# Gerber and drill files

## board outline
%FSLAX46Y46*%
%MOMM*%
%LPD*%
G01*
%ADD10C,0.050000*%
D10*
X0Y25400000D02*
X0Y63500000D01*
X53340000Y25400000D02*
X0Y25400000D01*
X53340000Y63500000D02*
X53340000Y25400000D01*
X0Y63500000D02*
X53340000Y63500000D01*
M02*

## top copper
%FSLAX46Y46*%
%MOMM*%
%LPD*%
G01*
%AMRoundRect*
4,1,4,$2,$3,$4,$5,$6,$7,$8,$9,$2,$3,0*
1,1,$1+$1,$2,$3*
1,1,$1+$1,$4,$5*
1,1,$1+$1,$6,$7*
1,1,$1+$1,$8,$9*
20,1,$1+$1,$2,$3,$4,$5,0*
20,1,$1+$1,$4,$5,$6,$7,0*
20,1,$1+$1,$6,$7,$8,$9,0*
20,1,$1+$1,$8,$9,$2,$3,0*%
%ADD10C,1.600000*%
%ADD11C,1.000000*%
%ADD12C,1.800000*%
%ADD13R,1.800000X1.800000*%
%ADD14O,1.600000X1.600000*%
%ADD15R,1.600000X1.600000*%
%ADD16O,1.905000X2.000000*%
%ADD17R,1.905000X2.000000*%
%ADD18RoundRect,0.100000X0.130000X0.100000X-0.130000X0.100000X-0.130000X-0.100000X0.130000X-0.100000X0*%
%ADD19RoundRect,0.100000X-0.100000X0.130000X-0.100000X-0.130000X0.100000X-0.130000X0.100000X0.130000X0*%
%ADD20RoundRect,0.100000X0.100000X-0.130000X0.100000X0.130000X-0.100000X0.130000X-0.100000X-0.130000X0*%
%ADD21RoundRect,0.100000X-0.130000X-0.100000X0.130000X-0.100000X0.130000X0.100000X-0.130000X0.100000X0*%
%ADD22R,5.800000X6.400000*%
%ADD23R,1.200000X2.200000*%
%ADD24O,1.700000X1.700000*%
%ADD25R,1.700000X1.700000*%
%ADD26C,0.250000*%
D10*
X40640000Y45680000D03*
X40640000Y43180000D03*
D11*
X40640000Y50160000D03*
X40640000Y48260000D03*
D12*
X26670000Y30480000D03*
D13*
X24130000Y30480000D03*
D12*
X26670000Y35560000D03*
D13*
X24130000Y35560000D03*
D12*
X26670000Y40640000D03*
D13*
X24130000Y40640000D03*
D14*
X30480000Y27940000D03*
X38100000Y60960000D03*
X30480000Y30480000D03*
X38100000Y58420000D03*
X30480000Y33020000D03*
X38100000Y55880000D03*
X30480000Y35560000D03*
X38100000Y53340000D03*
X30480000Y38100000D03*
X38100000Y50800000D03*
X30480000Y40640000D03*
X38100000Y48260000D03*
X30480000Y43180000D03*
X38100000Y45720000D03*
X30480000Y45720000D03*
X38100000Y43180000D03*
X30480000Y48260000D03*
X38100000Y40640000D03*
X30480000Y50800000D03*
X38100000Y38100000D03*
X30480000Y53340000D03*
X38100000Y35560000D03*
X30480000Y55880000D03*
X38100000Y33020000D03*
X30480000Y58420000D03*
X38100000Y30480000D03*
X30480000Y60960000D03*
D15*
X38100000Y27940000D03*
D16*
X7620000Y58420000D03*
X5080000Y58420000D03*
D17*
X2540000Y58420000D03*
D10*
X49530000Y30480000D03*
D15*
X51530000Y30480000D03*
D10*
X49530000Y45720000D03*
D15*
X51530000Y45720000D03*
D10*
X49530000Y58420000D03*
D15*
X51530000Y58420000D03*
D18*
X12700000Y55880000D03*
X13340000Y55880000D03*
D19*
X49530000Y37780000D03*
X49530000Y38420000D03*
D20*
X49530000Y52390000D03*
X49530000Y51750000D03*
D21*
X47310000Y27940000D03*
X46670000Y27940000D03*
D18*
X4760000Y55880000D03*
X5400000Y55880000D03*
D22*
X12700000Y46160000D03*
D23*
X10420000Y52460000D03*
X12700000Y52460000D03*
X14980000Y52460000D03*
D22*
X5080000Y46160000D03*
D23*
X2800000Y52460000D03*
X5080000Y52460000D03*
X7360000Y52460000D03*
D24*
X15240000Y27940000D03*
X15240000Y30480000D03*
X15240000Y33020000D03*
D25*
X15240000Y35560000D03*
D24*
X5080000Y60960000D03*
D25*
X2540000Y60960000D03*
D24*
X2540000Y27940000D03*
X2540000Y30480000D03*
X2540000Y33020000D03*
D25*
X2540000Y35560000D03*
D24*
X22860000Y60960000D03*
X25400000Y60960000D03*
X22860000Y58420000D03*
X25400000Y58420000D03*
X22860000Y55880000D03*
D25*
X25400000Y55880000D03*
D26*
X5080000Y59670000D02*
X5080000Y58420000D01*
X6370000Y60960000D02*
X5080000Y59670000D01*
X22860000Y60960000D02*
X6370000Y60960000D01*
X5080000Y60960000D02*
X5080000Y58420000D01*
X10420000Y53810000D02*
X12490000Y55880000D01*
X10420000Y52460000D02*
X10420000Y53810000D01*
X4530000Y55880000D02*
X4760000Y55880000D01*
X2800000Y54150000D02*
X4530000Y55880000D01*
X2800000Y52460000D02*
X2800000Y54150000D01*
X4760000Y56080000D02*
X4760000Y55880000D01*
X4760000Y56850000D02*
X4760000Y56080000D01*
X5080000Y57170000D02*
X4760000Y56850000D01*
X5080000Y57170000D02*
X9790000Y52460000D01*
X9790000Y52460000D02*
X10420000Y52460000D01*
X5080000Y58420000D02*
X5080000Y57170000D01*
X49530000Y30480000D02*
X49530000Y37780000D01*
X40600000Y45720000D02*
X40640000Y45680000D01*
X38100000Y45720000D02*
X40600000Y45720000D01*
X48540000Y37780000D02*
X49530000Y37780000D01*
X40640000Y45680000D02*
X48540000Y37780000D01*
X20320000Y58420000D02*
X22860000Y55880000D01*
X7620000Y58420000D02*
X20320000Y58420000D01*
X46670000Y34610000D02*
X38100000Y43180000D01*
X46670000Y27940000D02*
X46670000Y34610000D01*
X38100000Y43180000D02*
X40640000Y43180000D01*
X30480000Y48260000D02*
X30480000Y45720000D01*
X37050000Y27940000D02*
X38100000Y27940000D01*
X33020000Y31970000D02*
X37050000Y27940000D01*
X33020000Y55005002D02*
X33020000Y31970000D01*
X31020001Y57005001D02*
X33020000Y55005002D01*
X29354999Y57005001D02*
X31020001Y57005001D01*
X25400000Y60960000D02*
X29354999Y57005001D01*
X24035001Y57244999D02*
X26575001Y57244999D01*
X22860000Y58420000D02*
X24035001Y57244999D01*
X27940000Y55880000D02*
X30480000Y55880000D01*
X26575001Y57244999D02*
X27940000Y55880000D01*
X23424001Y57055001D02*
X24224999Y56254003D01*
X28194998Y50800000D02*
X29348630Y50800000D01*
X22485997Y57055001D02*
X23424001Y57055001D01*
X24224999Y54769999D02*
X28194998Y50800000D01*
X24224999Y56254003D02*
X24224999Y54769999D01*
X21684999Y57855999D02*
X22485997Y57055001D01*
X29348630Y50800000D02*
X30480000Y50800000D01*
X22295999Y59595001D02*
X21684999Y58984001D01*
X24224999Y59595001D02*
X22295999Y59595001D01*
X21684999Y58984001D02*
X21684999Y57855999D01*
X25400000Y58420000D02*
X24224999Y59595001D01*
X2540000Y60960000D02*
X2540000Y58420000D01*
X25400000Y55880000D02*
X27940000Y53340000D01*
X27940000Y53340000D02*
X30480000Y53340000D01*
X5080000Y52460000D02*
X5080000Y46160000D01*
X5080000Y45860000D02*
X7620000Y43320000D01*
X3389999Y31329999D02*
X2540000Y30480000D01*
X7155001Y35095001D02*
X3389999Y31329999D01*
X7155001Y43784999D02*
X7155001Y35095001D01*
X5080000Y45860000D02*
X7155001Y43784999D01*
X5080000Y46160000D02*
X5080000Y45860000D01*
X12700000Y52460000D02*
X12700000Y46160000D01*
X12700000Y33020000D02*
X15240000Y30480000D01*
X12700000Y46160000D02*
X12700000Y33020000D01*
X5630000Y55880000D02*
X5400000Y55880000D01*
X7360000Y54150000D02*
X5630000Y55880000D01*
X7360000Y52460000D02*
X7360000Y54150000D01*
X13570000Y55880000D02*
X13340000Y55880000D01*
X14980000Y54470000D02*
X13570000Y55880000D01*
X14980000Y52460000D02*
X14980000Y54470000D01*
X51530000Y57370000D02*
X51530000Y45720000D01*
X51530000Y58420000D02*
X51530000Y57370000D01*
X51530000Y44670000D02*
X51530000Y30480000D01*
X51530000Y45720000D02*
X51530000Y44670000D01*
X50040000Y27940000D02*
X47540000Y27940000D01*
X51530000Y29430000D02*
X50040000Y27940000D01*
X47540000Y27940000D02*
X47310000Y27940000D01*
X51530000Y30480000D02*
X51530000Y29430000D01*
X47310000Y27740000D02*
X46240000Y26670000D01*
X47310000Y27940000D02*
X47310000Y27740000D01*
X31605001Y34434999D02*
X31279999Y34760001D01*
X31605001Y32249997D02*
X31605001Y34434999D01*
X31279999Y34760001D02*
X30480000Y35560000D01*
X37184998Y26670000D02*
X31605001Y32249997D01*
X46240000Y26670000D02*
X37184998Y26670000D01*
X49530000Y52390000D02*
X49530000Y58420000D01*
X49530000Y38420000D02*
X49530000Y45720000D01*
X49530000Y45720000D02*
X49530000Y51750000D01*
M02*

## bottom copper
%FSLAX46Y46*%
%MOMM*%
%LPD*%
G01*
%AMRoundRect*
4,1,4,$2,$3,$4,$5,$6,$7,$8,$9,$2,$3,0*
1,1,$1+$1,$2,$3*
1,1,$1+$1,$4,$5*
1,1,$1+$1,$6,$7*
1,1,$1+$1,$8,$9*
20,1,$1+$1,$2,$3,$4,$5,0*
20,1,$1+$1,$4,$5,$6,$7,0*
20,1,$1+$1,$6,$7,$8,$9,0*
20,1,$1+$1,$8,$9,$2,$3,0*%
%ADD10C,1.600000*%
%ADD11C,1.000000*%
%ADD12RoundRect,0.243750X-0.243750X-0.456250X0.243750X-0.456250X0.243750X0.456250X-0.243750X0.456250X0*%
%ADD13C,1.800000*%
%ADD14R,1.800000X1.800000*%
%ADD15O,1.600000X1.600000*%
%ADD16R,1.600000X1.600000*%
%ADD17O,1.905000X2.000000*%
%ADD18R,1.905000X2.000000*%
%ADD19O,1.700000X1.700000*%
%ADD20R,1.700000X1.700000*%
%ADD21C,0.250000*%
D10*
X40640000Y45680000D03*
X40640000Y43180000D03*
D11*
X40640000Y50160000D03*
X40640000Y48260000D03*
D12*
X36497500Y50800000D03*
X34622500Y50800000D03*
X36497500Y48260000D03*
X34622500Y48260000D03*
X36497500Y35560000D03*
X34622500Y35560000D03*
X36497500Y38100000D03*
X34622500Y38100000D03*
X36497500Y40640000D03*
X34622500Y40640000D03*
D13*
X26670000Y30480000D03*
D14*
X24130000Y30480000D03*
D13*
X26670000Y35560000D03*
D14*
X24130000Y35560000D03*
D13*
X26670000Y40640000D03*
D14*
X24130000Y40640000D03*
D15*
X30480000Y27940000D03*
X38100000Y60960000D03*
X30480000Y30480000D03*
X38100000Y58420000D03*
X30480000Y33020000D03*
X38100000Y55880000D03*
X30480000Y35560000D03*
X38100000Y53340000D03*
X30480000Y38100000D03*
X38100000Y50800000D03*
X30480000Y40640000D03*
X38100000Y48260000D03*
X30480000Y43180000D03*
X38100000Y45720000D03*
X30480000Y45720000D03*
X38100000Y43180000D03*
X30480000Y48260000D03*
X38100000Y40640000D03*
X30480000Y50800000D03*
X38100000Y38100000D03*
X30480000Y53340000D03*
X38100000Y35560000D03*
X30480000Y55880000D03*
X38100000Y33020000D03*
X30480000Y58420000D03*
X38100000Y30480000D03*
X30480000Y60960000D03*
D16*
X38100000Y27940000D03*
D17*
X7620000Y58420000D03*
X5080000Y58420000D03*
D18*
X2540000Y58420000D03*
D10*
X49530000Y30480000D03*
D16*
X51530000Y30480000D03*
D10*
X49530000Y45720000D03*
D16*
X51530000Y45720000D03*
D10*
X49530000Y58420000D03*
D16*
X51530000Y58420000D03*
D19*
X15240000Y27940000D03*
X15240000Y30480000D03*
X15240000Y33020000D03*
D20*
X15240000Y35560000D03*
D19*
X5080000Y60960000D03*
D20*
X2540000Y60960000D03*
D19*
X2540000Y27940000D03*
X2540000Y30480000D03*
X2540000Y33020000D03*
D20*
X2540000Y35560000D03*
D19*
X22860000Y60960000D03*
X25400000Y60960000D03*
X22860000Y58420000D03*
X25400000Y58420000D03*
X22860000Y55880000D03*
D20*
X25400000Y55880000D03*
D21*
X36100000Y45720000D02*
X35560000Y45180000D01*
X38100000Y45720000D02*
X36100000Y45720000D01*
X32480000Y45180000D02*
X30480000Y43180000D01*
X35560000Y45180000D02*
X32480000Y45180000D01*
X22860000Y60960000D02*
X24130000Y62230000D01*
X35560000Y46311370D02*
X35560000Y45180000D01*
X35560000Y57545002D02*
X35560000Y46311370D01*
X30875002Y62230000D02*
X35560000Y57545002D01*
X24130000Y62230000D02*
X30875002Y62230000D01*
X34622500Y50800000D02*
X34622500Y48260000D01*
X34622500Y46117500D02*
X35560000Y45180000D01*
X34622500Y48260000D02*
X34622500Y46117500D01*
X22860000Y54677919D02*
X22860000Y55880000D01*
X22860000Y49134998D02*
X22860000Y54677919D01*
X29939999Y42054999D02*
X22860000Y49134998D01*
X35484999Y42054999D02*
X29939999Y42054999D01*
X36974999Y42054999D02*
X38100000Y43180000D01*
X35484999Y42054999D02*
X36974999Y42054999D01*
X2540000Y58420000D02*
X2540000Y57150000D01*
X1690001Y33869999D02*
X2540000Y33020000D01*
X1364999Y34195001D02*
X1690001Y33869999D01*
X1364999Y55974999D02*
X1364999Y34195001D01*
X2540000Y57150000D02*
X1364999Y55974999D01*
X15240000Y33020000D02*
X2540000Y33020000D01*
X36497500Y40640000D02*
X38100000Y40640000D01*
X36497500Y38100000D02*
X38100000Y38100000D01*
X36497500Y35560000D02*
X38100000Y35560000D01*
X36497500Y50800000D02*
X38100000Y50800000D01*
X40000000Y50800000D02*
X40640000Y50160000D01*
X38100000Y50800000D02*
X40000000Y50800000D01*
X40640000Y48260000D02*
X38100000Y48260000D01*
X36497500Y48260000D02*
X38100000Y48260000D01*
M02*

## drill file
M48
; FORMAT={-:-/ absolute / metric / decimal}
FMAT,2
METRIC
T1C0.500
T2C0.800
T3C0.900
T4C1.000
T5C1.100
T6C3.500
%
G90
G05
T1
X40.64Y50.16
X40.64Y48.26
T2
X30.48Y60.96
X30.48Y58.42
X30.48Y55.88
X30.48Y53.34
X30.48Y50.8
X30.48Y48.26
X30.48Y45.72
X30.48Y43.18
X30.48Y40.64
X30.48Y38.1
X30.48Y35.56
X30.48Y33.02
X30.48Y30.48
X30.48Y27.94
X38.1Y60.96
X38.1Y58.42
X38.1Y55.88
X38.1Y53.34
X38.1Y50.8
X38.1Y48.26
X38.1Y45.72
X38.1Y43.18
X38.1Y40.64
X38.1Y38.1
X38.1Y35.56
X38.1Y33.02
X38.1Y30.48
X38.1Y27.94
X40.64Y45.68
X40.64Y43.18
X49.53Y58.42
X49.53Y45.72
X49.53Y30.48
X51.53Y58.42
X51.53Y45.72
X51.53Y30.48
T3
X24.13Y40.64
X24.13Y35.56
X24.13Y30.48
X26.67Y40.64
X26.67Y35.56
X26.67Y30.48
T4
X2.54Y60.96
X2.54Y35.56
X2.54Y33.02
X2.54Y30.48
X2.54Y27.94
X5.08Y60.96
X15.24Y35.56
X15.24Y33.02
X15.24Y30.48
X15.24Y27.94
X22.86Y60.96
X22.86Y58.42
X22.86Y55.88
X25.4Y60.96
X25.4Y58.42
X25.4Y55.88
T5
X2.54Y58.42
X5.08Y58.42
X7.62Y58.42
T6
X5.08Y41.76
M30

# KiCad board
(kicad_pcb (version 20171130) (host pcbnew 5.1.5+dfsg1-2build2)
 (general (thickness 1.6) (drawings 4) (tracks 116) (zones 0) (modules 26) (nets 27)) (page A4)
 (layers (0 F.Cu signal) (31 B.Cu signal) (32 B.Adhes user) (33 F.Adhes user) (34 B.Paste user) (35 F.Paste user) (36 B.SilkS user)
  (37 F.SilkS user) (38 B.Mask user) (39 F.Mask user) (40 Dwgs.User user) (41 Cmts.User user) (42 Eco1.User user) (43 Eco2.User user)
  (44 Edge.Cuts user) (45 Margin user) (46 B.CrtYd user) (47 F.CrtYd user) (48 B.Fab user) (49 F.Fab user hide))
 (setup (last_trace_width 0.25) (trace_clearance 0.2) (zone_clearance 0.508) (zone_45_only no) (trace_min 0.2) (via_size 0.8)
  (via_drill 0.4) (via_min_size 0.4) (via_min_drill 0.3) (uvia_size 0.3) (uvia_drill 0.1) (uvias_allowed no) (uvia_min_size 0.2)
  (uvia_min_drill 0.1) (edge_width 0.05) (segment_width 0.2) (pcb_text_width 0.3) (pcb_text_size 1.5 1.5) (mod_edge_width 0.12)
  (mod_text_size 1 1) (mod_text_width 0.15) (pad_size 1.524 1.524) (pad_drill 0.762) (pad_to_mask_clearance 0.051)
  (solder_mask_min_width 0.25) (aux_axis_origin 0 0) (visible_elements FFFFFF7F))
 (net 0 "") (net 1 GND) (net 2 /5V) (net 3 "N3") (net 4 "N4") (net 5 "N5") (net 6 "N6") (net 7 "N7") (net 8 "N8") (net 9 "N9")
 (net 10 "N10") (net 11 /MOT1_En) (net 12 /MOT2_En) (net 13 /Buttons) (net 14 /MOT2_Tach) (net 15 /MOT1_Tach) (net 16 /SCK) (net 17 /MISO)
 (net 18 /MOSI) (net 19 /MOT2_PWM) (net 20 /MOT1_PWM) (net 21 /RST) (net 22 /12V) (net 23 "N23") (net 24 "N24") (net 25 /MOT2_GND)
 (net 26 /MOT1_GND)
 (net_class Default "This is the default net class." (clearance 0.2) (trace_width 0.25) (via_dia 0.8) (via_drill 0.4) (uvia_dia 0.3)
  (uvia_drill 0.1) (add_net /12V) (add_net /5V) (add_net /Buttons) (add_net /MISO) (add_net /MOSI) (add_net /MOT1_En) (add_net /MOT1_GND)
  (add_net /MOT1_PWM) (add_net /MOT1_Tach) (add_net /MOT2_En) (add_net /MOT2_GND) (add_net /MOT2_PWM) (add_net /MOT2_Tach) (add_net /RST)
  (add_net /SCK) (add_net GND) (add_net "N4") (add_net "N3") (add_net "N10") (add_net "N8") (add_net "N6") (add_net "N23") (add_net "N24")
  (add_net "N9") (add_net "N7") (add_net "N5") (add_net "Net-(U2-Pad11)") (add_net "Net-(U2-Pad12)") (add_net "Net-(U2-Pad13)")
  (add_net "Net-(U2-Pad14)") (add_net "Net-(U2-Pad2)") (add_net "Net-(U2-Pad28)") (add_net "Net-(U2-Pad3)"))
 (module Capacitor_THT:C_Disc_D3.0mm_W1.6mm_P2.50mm (layer F.Cu) (at 40.64 -43.18 90)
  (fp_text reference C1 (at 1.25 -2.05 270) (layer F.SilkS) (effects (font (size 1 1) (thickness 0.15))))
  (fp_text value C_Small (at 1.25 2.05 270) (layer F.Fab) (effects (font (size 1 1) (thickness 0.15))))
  (pad 2 thru_hole circle (at 2.5 0 90) (size 1.6 1.6) (drill 0.8) (layers *.Cu *.Mask) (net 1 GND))
  (pad 1 thru_hole circle (at 0 0 90) (size 1.6 1.6) (drill 0.8) (layers *.Cu *.Mask) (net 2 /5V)))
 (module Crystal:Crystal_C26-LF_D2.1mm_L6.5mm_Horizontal (layer F.Cu) (at 40.64 -48.26 90)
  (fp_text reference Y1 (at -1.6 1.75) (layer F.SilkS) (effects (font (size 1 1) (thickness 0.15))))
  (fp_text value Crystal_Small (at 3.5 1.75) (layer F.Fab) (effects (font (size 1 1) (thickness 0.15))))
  (pad 2 thru_hole circle (at 1.9 0 90) (size 1 1) (drill 0.5) (layers *.Cu *.Mask) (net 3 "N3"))
  (pad 1 thru_hole circle (at 0 0 90) (size 1 1) (drill 0.5) (layers *.Cu *.Mask) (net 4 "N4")))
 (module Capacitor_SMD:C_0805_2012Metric (layer B.Cu) (at 35.56 -50.8)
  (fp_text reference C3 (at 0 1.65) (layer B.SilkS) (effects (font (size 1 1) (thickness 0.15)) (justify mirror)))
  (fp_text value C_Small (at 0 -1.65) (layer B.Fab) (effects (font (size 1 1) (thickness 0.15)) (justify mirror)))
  (pad 2 smd roundrect (at 0.9375 0) (size 0.975 1.4) (layers B.Cu B.Paste B.Mask) (roundrect_rratio 0.25) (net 3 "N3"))
  (pad 1 smd roundrect (at -0.9375 0) (size 0.975 1.4) (layers B.Cu B.Paste B.Mask) (roundrect_rratio 0.25) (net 1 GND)))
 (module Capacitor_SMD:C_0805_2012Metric (layer B.Cu) (at 35.56 -48.26)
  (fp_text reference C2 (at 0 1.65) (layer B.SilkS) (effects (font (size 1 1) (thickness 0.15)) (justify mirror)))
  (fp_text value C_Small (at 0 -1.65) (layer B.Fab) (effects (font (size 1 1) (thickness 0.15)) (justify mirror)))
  (pad 2 smd roundrect (at 0.9375 0) (size 0.975 1.4) (layers B.Cu B.Paste B.Mask) (roundrect_rratio 0.25) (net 4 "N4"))
  (pad 1 smd roundrect (at -0.9375 0) (size 0.975 1.4) (layers B.Cu B.Paste B.Mask) (roundrect_rratio 0.25) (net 1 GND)))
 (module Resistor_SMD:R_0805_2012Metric (layer B.Cu) (at 35.56 -35.56)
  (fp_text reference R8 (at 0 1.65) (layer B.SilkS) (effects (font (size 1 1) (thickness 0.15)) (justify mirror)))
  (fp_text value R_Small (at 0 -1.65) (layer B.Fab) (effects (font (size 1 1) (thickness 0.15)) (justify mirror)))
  (pad 2 smd roundrect (at 0.9375 0) (size 0.975 1.4) (layers B.Cu B.Paste B.Mask) (roundrect_rratio 0.25) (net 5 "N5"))
  (pad 1 smd roundrect (at -0.9375 0) (size 0.975 1.4) (layers B.Cu B.Paste B.Mask) (roundrect_rratio 0.25) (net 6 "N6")))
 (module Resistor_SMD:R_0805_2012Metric (layer B.Cu) (at 35.56 -38.1)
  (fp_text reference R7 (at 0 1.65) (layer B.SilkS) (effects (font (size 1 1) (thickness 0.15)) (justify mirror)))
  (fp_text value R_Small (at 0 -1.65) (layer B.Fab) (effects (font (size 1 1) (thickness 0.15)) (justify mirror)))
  (pad 2 smd roundrect (at 0.9375 0) (size 0.975 1.4) (layers B.Cu B.Paste B.Mask) (roundrect_rratio 0.25) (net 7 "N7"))
  (pad 1 smd roundrect (at -0.9375 0) (size 0.975 1.4) (layers B.Cu B.Paste B.Mask) (roundrect_rratio 0.25) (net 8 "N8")))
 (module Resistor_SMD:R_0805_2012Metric (layer B.Cu) (at 35.56 -40.64)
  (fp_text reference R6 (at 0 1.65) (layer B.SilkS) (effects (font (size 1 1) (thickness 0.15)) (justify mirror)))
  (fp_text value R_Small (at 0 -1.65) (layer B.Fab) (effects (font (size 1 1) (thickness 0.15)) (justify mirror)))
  (pad 2 smd roundrect (at 0.9375 0) (size 0.975 1.4) (layers B.Cu B.Paste B.Mask) (roundrect_rratio 0.25) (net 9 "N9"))
  (pad 1 smd roundrect (at -0.9375 0) (size 0.975 1.4) (layers B.Cu B.Paste B.Mask) (roundrect_rratio 0.25) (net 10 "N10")))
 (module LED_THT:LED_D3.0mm (layer B.Cu) (at 24.13 -30.48)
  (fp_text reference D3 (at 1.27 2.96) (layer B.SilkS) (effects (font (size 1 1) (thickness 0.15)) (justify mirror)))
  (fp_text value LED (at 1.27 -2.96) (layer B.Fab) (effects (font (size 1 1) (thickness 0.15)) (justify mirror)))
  (pad 2 thru_hole circle (at 2.54 0) (size 1.8 1.8) (drill 0.9) (layers *.Cu *.Mask) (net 6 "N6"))
  (pad 1 thru_hole rect (at 0 0) (size 1.8 1.8) (drill 0.9) (layers *.Cu *.Mask) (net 1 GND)))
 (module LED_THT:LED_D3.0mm (layer B.Cu) (at 24.13 -35.56)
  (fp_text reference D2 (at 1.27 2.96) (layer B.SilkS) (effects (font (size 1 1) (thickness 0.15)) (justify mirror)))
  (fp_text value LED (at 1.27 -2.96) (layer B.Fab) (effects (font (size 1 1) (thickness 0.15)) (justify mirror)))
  (pad 2 thru_hole circle (at 2.54 0) (size 1.8 1.8) (drill 0.9) (layers *.Cu *.Mask) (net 8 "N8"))
  (pad 1 thru_hole rect (at 0 0) (size 1.8 1.8) (drill 0.9) (layers *.Cu *.Mask) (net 1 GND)))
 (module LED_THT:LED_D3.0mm (layer B.Cu) (at 24.13 -40.64)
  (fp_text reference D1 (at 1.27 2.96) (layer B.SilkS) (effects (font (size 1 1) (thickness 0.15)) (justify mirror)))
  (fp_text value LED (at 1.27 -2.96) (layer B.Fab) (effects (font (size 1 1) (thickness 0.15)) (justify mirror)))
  (pad 2 thru_hole circle (at 2.54 0) (size 1.8 1.8) (drill 0.9) (layers *.Cu *.Mask) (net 10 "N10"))
  (pad 1 thru_hole rect (at 0 0) (size 1.8 1.8) (drill 0.9) (layers *.Cu *.Mask) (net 1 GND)))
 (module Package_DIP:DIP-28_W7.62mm (layer F.Cu) (at 38.1 -27.94 180)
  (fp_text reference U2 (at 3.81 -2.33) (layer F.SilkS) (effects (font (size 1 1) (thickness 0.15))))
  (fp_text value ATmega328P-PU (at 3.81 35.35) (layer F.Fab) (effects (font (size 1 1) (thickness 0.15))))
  (pad 28 thru_hole oval (at 7.62 0 180) (size 1.6 1.6) (drill 0.8) (layers *.Cu *.Mask))
  (pad 14 thru_hole oval (at 0 33.02 180) (size 1.6 1.6) (drill 0.8) (layers *.Cu *.Mask))
  (pad 27 thru_hole oval (at 7.62 2.54 180) (size 1.6 1.6) (drill 0.8) (layers *.Cu *.Mask) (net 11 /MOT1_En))
  (pad 13 thru_hole oval (at 0 30.48 180) (size 1.6 1.6) (drill 0.8) (layers *.Cu *.Mask))
  (pad 26 thru_hole oval (at 7.62 5.08 180) (size 1.6 1.6) (drill 0.8) (layers *.Cu *.Mask) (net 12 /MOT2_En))
  (pad 12 thru_hole oval (at 0 27.94 180) (size 1.6 1.6) (drill 0.8) (layers *.Cu *.Mask))
  (pad 25 thru_hole oval (at 7.62 7.62 180) (size 1.6 1.6) (drill 0.8) (layers *.Cu *.Mask) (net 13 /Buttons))
  (pad 11 thru_hole oval (at 0 25.4 180) (size 1.6 1.6) (drill 0.8) (layers *.Cu *.Mask))
  (pad 24 thru_hole oval (at 7.62 10.16 180) (size 1.6 1.6) (drill 0.8) (layers *.Cu *.Mask) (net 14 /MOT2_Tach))
  (pad 10 thru_hole oval (at 0 22.86 180) (size 1.6 1.6) (drill 0.8) (layers *.Cu *.Mask) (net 3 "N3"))
  (pad 23 thru_hole oval (at 7.62 12.7 180) (size 1.6 1.6) (drill 0.8) (layers *.Cu *.Mask) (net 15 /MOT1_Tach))
  (pad 9 thru_hole oval (at 0 20.32 180) (size 1.6 1.6) (drill 0.8) (layers *.Cu *.Mask) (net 4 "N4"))
  (pad 22 thru_hole oval (at 7.62 15.24 180) (size 1.6 1.6) (drill 0.8) (layers *.Cu *.Mask) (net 1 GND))
  (pad 8 thru_hole oval (at 0 17.78 180) (size 1.6 1.6) (drill 0.8) (layers *.Cu *.Mask) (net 1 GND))
  (pad 21 thru_hole oval (at 7.62 17.78 180) (size 1.6 1.6) (drill 0.8) (layers *.Cu *.Mask) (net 2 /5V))
  (pad 7 thru_hole oval (at 0 15.24 180) (size 1.6 1.6) (drill 0.8) (layers *.Cu *.Mask) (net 2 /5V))
  (pad 20 thru_hole oval (at 7.62 20.32 180) (size 1.6 1.6) (drill 0.8) (layers *.Cu *.Mask) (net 2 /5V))
  (pad 6 thru_hole oval (at 0 12.7 180) (size 1.6 1.6) (drill 0.8) (layers *.Cu *.Mask) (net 9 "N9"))
  (pad 19 thru_hole oval (at 7.62 22.86 180) (size 1.6 1.6) (drill 0.8) (layers *.Cu *.Mask) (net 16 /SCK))
  (pad 5 thru_hole oval (at 0 10.16 180) (size 1.6 1.6) (drill 0.8) (layers *.Cu *.Mask) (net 7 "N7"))
  (pad 18 thru_hole oval (at 7.62 25.4 180) (size 1.6 1.6) (drill 0.8) (layers *.Cu *.Mask) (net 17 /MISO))
  (pad 4 thru_hole oval (at 0 7.62 180) (size 1.6 1.6) (drill 0.8) (layers *.Cu *.Mask) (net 5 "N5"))
  (pad 17 thru_hole oval (at 7.62 27.94 180) (size 1.6 1.6) (drill 0.8) (layers *.Cu *.Mask) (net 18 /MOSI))
  (pad 3 thru_hole oval (at 0 5.08 180) (size 1.6 1.6) (drill 0.8) (layers *.Cu *.Mask))
  (pad 16 thru_hole oval (at 7.62 30.48 180) (size 1.6 1.6) (drill 0.8) (layers *.Cu *.Mask) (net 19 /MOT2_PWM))
  (pad 2 thru_hole oval (at 0 2.54 180) (size 1.6 1.6) (drill 0.8) (layers *.Cu *.Mask))
  (pad 15 thru_hole oval (at 7.62 33.02 180) (size 1.6 1.6) (drill 0.8) (layers *.Cu *.Mask) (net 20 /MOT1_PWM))
  (pad 1 thru_hole rect (at 0 0 180) (size 1.6 1.6) (drill 0.8) (layers *.Cu *.Mask) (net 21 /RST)))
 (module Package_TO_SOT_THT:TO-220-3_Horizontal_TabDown (layer B.Cu) (at 2.54 -58.42)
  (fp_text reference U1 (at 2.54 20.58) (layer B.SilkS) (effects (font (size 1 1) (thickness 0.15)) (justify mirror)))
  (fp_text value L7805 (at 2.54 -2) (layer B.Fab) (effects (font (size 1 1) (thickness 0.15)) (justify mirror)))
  (pad 3 thru_hole oval (at 5.08 0) (size 1.905 2) (drill 1.1) (layers *.Cu *.Mask) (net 2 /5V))
  (pad 2 thru_hole oval (at 2.54 0) (size 1.905 2) (drill 1.1) (layers *.Cu *.Mask) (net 1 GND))
  (pad 1 thru_hole rect (at 0 0) (size 1.905 2) (drill 1.1) (layers *.Cu *.Mask) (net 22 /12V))
  (pad "" np_thru_hole oval (at 2.54 16.66) (size 3.5 3.5) (drill 3.5) (layers *.Cu *.Mask)))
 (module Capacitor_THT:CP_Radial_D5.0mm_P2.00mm (layer B.Cu) (at 51.53 -30.48 180)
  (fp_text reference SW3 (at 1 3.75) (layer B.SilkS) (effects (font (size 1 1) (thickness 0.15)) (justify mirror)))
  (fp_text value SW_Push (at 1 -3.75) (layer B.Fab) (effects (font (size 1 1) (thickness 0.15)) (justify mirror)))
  (pad 2 thru_hole circle (at 2 0 180) (size 1.6 1.6) (drill 0.8) (layers *.Cu *.Mask) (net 1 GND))
  (pad 1 thru_hole rect (at 0 0 180) (size 1.6 1.6) (drill 0.8) (layers *.Cu *.Mask) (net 13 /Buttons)))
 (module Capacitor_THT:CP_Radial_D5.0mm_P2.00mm (layer B.Cu) (at 51.53 -45.72 180)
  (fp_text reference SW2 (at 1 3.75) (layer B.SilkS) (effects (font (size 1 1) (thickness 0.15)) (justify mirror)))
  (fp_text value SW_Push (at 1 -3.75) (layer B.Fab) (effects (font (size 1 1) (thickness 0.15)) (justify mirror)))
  (pad 2 thru_hole circle (at 2 0 180) (size 1.6 1.6) (drill 0.8) (layers *.Cu *.Mask) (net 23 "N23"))
  (pad 1 thru_hole rect (at 0 0 180) (size 1.6 1.6) (drill 0.8) (layers *.Cu *.Mask) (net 13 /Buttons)))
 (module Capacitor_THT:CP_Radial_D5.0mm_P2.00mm (layer B.Cu) (at 51.53 -58.42 180)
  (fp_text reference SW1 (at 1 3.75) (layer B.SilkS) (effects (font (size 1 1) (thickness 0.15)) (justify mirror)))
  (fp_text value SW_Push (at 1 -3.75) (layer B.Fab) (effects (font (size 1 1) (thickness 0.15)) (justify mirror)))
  (pad 2 thru_hole circle (at 2 0 180) (size 1.6 1.6) (drill 0.8) (layers *.Cu *.Mask) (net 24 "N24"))
  (pad 1 thru_hole rect (at 0 0 180) (size 1.6 1.6) (drill 0.8) (layers *.Cu *.Mask) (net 13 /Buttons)))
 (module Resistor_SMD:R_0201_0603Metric (layer F.Cu) (at 13.02 -55.88 180)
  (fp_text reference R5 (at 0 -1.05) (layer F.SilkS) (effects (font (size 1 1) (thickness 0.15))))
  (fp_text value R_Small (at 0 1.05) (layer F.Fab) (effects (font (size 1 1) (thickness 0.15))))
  (pad 2 smd roundrect (at 0.32 0 180) (size 0.46 0.4) (layers F.Cu F.Mask) (roundrect_rratio 0.25) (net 1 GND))
  (pad 1 smd roundrect (at -0.32 0 180) (size 0.46 0.4) (layers F.Cu F.Mask) (roundrect_rratio 0.25) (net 12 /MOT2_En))
  (pad "" smd roundrect (at 0.345 0 180) (size 0.318 0.36) (layers F.Paste) (roundrect_rratio 0.25))
  (pad "" smd roundrect (at -0.345 0 180) (size 0.318 0.36) (layers F.Paste) (roundrect_rratio 0.25)))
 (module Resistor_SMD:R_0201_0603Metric (layer F.Cu) (at 49.53 -38.1 270)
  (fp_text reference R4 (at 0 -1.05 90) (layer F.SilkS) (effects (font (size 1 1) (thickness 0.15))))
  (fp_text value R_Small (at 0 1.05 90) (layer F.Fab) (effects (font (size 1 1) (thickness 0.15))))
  (pad 2 smd roundrect (at 0.32 0 270) (size 0.46 0.4) (layers F.Cu F.Mask) (roundrect_rratio 0.25) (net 1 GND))
  (pad 1 smd roundrect (at -0.32 0 270) (size 0.46 0.4) (layers F.Cu F.Mask) (roundrect_rratio 0.25) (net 23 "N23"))
  (pad "" smd roundrect (at 0.345 0 270) (size 0.318 0.36) (layers F.Paste) (roundrect_rratio 0.25))
  (pad "" smd roundrect (at -0.345 0 270) (size 0.318 0.36) (layers F.Paste) (roundrect_rratio 0.25)))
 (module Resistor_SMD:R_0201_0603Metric (layer F.Cu) (at 49.53 -52.07 90)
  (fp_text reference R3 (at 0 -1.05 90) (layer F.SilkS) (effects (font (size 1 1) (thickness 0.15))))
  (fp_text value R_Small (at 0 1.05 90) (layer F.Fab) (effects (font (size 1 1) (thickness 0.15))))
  (pad 2 smd roundrect (at 0.32 0 90) (size 0.46 0.4) (layers F.Cu F.Mask) (roundrect_rratio 0.25) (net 24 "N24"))
  (pad 1 smd roundrect (at -0.32 0 90) (size 0.46 0.4) (layers F.Cu F.Mask) (roundrect_rratio 0.25) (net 23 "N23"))
  (pad "" smd roundrect (at 0.345 0 90) (size 0.318 0.36) (layers F.Paste) (roundrect_rratio 0.25))
  (pad "" smd roundrect (at -0.345 0 90) (size 0.318 0.36) (layers F.Paste) (roundrect_rratio 0.25)))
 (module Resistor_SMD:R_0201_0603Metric (layer F.Cu) (at 46.99 -27.94)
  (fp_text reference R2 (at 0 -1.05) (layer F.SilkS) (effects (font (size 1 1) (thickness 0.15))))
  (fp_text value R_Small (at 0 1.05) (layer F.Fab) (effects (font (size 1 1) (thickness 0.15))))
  (pad 2 smd roundrect (at 0.32 0) (size 0.46 0.4) (layers F.Cu F.Mask) (roundrect_rratio 0.25) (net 13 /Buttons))
  (pad 1 smd roundrect (at -0.32 0) (size 0.46 0.4) (layers F.Cu F.Mask) (roundrect_rratio 0.25) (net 2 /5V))
  (pad "" smd roundrect (at 0.345 0) (size 0.318 0.36) (layers F.Paste) (roundrect_rratio 0.25))
  (pad "" smd roundrect (at -0.345 0) (size 0.318 0.36) (layers F.Paste) (roundrect_rratio 0.25)))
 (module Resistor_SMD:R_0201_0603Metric (layer F.Cu) (at 5.08 -55.88 180)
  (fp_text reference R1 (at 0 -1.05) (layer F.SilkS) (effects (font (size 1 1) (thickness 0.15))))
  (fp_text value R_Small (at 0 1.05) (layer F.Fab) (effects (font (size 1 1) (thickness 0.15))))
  (pad 2 smd roundrect (at 0.32 0 180) (size 0.46 0.4) (layers F.Cu F.Mask) (roundrect_rratio 0.25) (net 1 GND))
  (pad 1 smd roundrect (at -0.32 0 180) (size 0.46 0.4) (layers F.Cu F.Mask) (roundrect_rratio 0.25) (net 11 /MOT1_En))
  (pad "" smd roundrect (at 0.345 0 180) (size 0.318 0.36) (layers F.Paste) (roundrect_rratio 0.25))
  (pad "" smd roundrect (at -0.345 0 180) (size 0.318 0.36) (layers F.Paste) (roundrect_rratio 0.25)))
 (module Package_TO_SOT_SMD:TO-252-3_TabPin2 (layer F.Cu) (at 12.7 -48.26 270)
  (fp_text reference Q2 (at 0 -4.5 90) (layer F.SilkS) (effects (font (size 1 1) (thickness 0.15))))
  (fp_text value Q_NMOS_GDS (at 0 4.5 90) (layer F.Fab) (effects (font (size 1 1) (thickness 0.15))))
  (pad "" smd rect (at 0.425 1.525 270) (size 3.05 2.75) (layers F.Paste))
  (pad "" smd rect (at 3.775 -1.525 270) (size 3.05 2.75) (layers F.Paste))
  (pad "" smd rect (at 0.425 -1.525 270) (size 3.05 2.75) (layers F.Paste))
  (pad "" smd rect (at 3.775 1.525 270) (size 3.05 2.75) (layers F.Paste))
  (pad 2 smd rect (at 2.1 0 270) (size 6.4 5.8) (layers F.Cu F.Mask) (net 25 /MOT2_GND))
  (pad 3 smd rect (at -4.2 2.28 270) (size 2.2 1.2) (layers F.Cu F.Paste F.Mask) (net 1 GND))
  (pad 2 smd rect (at -4.2 0 270) (size 2.2 1.2) (layers F.Cu F.Paste F.Mask) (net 25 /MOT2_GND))
  (pad 1 smd rect (at -4.2 -2.28 270) (size 2.2 1.2) (layers F.Cu F.Paste F.Mask) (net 12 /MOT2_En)))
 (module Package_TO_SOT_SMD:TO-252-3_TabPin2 (layer F.Cu) (at 5.08 -48.26 270)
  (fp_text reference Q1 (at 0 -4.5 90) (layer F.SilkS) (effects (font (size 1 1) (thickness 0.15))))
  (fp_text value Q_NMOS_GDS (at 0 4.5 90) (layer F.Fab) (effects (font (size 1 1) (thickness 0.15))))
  (pad "" smd rect (at 0.425 1.525 270) (size 3.05 2.75) (layers F.Paste))
  (pad "" smd rect (at 3.775 -1.525 270) (size 3.05 2.75) (layers F.Paste))
  (pad "" smd rect (at 0.425 -1.525 270) (size 3.05 2.75) (layers F.Paste))
  (pad "" smd rect (at 3.775 1.525 270) (size 3.05 2.75) (layers F.Paste))
  (pad 2 smd rect (at 2.1 0 270) (size 6.4 5.8) (layers F.Cu F.Mask) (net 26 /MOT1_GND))
  (pad 3 smd rect (at -4.2 2.28 270) (size 2.2 1.2) (layers F.Cu F.Paste F.Mask) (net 1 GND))
  (pad 2 smd rect (at -4.2 0 270) (size 2.2 1.2) (layers F.Cu F.Paste F.Mask) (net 26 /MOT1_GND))
  (pad 1 smd rect (at -4.2 -2.28 270) (size 2.2 1.2) (layers F.Cu F.Paste F.Mask) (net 11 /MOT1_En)))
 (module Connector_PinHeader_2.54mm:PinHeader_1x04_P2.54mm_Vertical (layer F.Cu) (at 15.24 -35.56)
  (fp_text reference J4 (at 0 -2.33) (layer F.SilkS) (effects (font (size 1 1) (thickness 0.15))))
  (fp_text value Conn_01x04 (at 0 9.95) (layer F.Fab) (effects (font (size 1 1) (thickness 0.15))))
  (pad 4 thru_hole oval (at 0 7.62) (size 1.7 1.7) (drill 1) (layers *.Cu *.Mask) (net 19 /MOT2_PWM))
  (pad 3 thru_hole oval (at 0 5.08) (size 1.7 1.7) (drill 1) (layers *.Cu *.Mask) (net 25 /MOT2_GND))
  (pad 2 thru_hole oval (at 0 2.54) (size 1.7 1.7) (drill 1) (layers *.Cu *.Mask) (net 22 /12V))
  (pad 1 thru_hole rect (at 0 0) (size 1.7 1.7) (drill 1) (layers *.Cu *.Mask) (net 14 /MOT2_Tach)))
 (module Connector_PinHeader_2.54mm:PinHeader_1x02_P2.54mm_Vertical (layer F.Cu) (at 2.54 -60.96 90)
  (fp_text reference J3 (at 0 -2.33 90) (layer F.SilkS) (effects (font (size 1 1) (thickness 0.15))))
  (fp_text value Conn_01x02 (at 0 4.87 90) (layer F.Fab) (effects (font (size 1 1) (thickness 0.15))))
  (pad 2 thru_hole oval (at 0 2.54 90) (size 1.7 1.7) (drill 1) (layers *.Cu *.Mask) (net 1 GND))
  (pad 1 thru_hole rect (at 0 0 90) (size 1.7 1.7) (drill 1) (layers *.Cu *.Mask) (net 22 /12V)))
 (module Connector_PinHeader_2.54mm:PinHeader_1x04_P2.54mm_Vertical (layer F.Cu) (at 2.54 -35.56)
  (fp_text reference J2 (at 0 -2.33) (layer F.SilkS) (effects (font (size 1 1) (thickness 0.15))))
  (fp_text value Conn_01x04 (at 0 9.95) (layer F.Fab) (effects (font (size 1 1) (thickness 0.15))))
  (pad 4 thru_hole oval (at 0 7.62) (size 1.7 1.7) (drill 1) (layers *.Cu *.Mask) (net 20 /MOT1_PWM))
  (pad 3 thru_hole oval (at 0 5.08) (size 1.7 1.7) (drill 1) (layers *.Cu *.Mask) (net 26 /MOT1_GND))
  (pad 2 thru_hole oval (at 0 2.54) (size 1.7 1.7) (drill 1) (layers *.Cu *.Mask) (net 22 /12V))
  (pad 1 thru_hole rect (at 0 0) (size 1.7 1.7) (drill 1) (layers *.Cu *.Mask) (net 15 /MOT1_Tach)))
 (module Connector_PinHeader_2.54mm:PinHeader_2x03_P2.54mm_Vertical (layer F.Cu) (at 25.4 -55.88 180)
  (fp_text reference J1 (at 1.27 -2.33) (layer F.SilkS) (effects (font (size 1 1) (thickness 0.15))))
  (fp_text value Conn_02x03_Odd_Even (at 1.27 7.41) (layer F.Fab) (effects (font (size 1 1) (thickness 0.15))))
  (pad 6 thru_hole oval (at 2.54 5.08 180) (size 1.7 1.7) (drill 1) (layers *.Cu *.Mask) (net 1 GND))
  (pad 5 thru_hole oval (at 0 5.08 180) (size 1.7 1.7) (drill 1) (layers *.Cu *.Mask) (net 21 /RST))
  (pad 4 thru_hole oval (at 2.54 2.54 180) (size 1.7 1.7) (drill 1) (layers *.Cu *.Mask) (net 18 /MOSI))
  (pad 3 thru_hole oval (at 0 2.54 180) (size 1.7 1.7) (drill 1) (layers *.Cu *.Mask) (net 16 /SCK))
  (pad 2 thru_hole oval (at 2.54 0 180) (size 1.7 1.7) (drill 1) (layers *.Cu *.Mask) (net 2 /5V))
  (pad 1 thru_hole rect (at 0 0 180) (size 1.7 1.7) (drill 1) (layers *.Cu *.Mask) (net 17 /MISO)))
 (gr_line (start 0 -25.4) (end 0 -63.5) (layer Edge.Cuts) (width 0.05))
 (gr_line (start 53.34 -25.4) (end 0 -25.4) (layer Edge.Cuts) (width 0.05))
 (gr_line (start 53.34 -63.5) (end 53.34 -25.4) (layer Edge.Cuts) (width 0.05))
 (gr_line (start 0 -63.5) (end 53.34 -63.5) (layer Edge.Cuts) (width 0.05))
 (segment (start 5.08 -59.67) (end 5.08 -58.42) (width 0.25) (layer F.Cu) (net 1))
 (segment (start 6.37 -60.96) (end 5.08 -59.67) (width 0.25) (layer F.Cu) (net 1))
 (segment (start 22.86 -60.96) (end 6.37 -60.96) (width 0.25) (layer F.Cu) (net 1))
 (segment (start 5.08 -60.96) (end 5.08 -58.42) (width 0.25) (layer F.Cu) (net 1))
 (segment (start 10.42 -53.81) (end 12.49 -55.88) (width 0.25) (layer F.Cu) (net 1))
 (segment (start 10.42 -52.46) (end 10.42 -53.81) (width 0.25) (layer F.Cu) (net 1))
 (segment (start 4.53 -55.88) (end 4.76 -55.88) (width 0.25) (layer F.Cu) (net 1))
 (segment (start 2.8 -54.15) (end 4.53 -55.88) (width 0.25) (layer F.Cu) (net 1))
 (segment (start 2.8 -52.46) (end 2.8 -54.15) (width 0.25) (layer F.Cu) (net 1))
 (segment (start 4.76 -56.08) (end 4.76 -55.88) (width 0.25) (layer F.Cu) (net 1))
 (segment (start 4.76 -56.85) (end 4.76 -56.08) (width 0.25) (layer F.Cu) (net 1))
 (segment (start 5.08 -57.17) (end 4.76 -56.85) (width 0.25) (layer F.Cu) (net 1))
 (segment (start 5.08 -57.17) (end 9.79 -52.46) (width 0.25) (layer F.Cu) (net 1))
 (segment (start 9.79 -52.46) (end 10.42 -52.46) (width 0.25) (layer F.Cu) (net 1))
 (segment (start 5.08 -58.42) (end 5.08 -57.17) (width 0.25) (layer F.Cu) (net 1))
 (segment (start 36.1 -45.72) (end 35.56 -45.18) (width 0.25) (layer B.Cu) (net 1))
 (segment (start 38.1 -45.72) (end 36.1 -45.72) (width 0.25) (layer B.Cu) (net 1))
 (segment (start 32.48 -45.18) (end 30.48 -43.18) (width 0.25) (layer B.Cu) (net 1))
 (segment (start 35.56 -45.18) (end 32.48 -45.18) (width 0.25) (layer B.Cu) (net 1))
 (segment (start 22.86 -60.96) (end 24.13 -62.23) (width 0.25) (layer B.Cu) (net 1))
 (segment (start 35.56 -46.31137) (end 35.56 -45.18) (width 0.25) (layer B.Cu) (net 1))
 (segment (start 35.56 -57.545002) (end 35.56 -46.31137) (width 0.25) (layer B.Cu) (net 1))
 (segment (start 30.875002 -62.23) (end 35.56 -57.545002) (width 0.25) (layer B.Cu) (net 1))
 (segment (start 24.13 -62.23) (end 30.875002 -62.23) (width 0.25) (layer B.Cu) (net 1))
 (segment (start 49.53 -30.48) (end 49.53 -37.78) (width 0.25) (layer F.Cu) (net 1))
 (segment (start 40.6 -45.72) (end 40.64 -45.68) (width 0.25) (layer F.Cu) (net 1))
 (segment (start 38.1 -45.72) (end 40.6 -45.72) (width 0.25) (layer F.Cu) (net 1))
 (segment (start 48.54 -37.78) (end 49.53 -37.78) (width 0.25) (layer F.Cu) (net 1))
 (segment (start 40.64 -45.68) (end 48.54 -37.78) (width 0.25) (layer F.Cu) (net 1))
 (segment (start 34.6225 -50.8) (end 34.6225 -48.26) (width 0.25) (layer B.Cu) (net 1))
 (segment (start 34.6225 -46.1175) (end 35.56 -45.18) (width 0.25) (layer B.Cu) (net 1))
 (segment (start 34.6225 -48.26) (end 34.6225 -46.1175) (width 0.25) (layer B.Cu) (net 1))
 (segment (start 20.32 -58.42) (end 22.86 -55.88) (width 0.25) (layer F.Cu) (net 2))
 (segment (start 7.62 -58.42) (end 20.32 -58.42) (width 0.25) (layer F.Cu) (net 2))
 (segment (start 22.86 -54.677919) (end 22.86 -55.88) (width 0.25) (layer B.Cu) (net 2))
 (segment (start 22.86 -49.134998) (end 22.86 -54.677919) (width 0.25) (layer B.Cu) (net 2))
 (segment (start 29.939999 -42.054999) (end 22.86 -49.134998) (width 0.25) (layer B.Cu) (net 2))
 (segment (start 35.484999 -42.054999) (end 29.939999 -42.054999) (width 0.25) (layer B.Cu) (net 2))
 (segment (start 46.67 -34.61) (end 38.1 -43.18) (width 0.25) (layer F.Cu) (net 2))
 (segment (start 46.67 -27.94) (end 46.67 -34.61) (width 0.25) (layer F.Cu) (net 2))
 (segment (start 38.1 -43.18) (end 40.64 -43.18) (width 0.25) (layer F.Cu) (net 2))
 (segment (start 36.974999 -42.054999) (end 38.1 -43.18) (width 0.25) (layer B.Cu) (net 2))
 (segment (start 35.484999 -42.054999) (end 36.974999 -42.054999) (width 0.25) (layer B.Cu) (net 2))
 (segment (start 30.48 -48.26) (end 30.48 -45.72) (width 0.25) (layer F.Cu) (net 2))
 (segment (start 37.05 -27.94) (end 38.1 -27.94) (width 0.25) (layer F.Cu) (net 21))
 (segment (start 33.02 -31.97) (end 37.05 -27.94) (width 0.25) (layer F.Cu) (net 21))
 (segment (start 33.02 -55.005002) (end 33.02 -31.97) (width 0.25) (layer F.Cu) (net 21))
 (segment (start 31.020001 -57.005001) (end 33.02 -55.005002) (width 0.25) (layer F.Cu) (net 21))
 (segment (start 29.354999 -57.005001) (end 31.020001 -57.005001) (width 0.25) (layer F.Cu) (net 21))
 (segment (start 25.4 -60.96) (end 29.354999 -57.005001) (width 0.25) (layer F.Cu) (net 21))
 (segment (start 24.035001 -57.244999) (end 26.575001 -57.244999) (width 0.25) (layer F.Cu) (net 18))
 (segment (start 22.86 -58.42) (end 24.035001 -57.244999) (width 0.25) (layer F.Cu) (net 18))
 (segment (start 27.94 -55.88) (end 30.48 -55.88) (width 0.25) (layer F.Cu) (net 18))
 (segment (start 26.575001 -57.244999) (end 27.94 -55.88) (width 0.25) (layer F.Cu) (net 18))
 (segment (start 23.424001 -57.055001) (end 24.224999 -56.254003) (width 0.25) (layer F.Cu) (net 16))
 (segment (start 28.194998 -50.8) (end 29.34863 -50.8) (width 0.25) (layer F.Cu) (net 16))
 (segment (start 22.485997 -57.055001) (end 23.424001 -57.055001) (width 0.25) (layer F.Cu) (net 16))
 (segment (start 24.224999 -54.769999) (end 28.194998 -50.8) (width 0.25) (layer F.Cu) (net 16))
 (segment (start 24.224999 -56.254003) (end 24.224999 -54.769999) (width 0.25) (layer F.Cu) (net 16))
 (segment (start 21.684999 -57.855999) (end 22.485997 -57.055001) (width 0.25) (layer F.Cu) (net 16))
 (segment (start 29.34863 -50.8) (end 30.48 -50.8) (width 0.25) (layer F.Cu) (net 16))
 (segment (start 22.295999 -59.595001) (end 21.684999 -58.984001) (width 0.25) (layer F.Cu) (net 16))
 (segment (start 24.224999 -59.595001) (end 22.295999 -59.595001) (width 0.25) (layer F.Cu) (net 16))
 (segment (start 21.684999 -58.984001) (end 21.684999 -57.855999) (width 0.25) (layer F.Cu) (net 16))
 (segment (start 25.4 -58.42) (end 24.224999 -59.595001) (width 0.25) (layer F.Cu) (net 16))
 (segment (start 2.54 -60.96) (end 2.54 -58.42) (width 0.25) (layer F.Cu) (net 22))
 (segment (start 2.54 -58.42) (end 2.54 -57.15) (width 0.25) (layer B.Cu) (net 22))
 (segment (start 1.690001 -33.869999) (end 2.54 -33.02) (width 0.25) (layer B.Cu) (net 22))
 (segment (start 1.364999 -34.195001) (end 1.690001 -33.869999) (width 0.25) (layer B.Cu) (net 22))
 (segment (start 1.364999 -55.974999) (end 1.364999 -34.195001) (width 0.25) (layer B.Cu) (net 22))
 (segment (start 2.54 -57.15) (end 1.364999 -55.974999) (width 0.25) (layer B.Cu) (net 22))
 (segment (start 15.24 -33.02) (end 2.54 -33.02) (width 0.25) (layer B.Cu) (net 22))
 (segment (start 25.4 -55.88) (end 27.94 -53.34) (width 0.25) (layer F.Cu) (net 17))
 (segment (start 27.94 -53.34) (end 30.48 -53.34) (width 0.25) (layer F.Cu) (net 17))
 (segment (start 5.08 -52.46) (end 5.08 -46.16) (width 0.25) (layer F.Cu) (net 26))
 (segment (start 5.08 -45.86) (end 7.62 -43.32) (width 0.25) (layer F.Cu) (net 26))
 (segment (start 3.389999 -31.329999) (end 2.54 -30.48) (width 0.25) (layer F.Cu) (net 26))
 (segment (start 7.155001 -35.095001) (end 3.389999 -31.329999) (width 0.25) (layer F.Cu) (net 26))
 (segment (start 7.155001 -43.784999) (end 7.155001 -35.095001) (width 0.25) (layer F.Cu) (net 26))
 (segment (start 5.08 -45.86) (end 7.155001 -43.784999) (width 0.25) (layer F.Cu) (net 26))
 (segment (start 5.08 -46.16) (end 5.08 -45.86) (width 0.25) (layer F.Cu) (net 26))
 (segment (start 12.7 -52.46) (end 12.7 -46.16) (width 0.25) (layer F.Cu) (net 25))
 (segment (start 12.7 -33.02) (end 15.24 -30.48) (width 0.25) (layer F.Cu) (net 25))
 (segment (start 12.7 -46.16) (end 12.7 -33.02) (width 0.25) (layer F.Cu) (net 25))
 (segment (start 5.63 -55.88) (end 5.4 -55.88) (width 0.25) (layer F.Cu) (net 11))
 (segment (start 7.36 -54.15) (end 5.63 -55.88) (width 0.25) (layer F.Cu) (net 11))
 (segment (start 7.36 -52.46) (end 7.36 -54.15) (width 0.25) (layer F.Cu) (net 11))
 (segment (start 13.57 -55.88) (end 13.34 -55.88) (width 0.25) (layer F.Cu) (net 12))
 (segment (start 14.98 -54.47) (end 13.57 -55.88) (width 0.25) (layer F.Cu) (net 12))
 (segment (start 14.98 -52.46) (end 14.98 -54.47) (width 0.25) (layer F.Cu) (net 12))
 (segment (start 51.53 -57.37) (end 51.53 -45.72) (width 0.25) (layer F.Cu) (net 13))
 (segment (start 51.53 -58.42) (end 51.53 -57.37) (width 0.25) (layer F.Cu) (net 13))
 (segment (start 51.53 -44.67) (end 51.53 -30.48) (width 0.25) (layer F.Cu) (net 13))
 (segment (start 51.53 -45.72) (end 51.53 -44.67) (width 0.25) (layer F.Cu) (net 13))
 (segment (start 50.04 -27.94) (end 47.54 -27.94) (width 0.25) (layer F.Cu) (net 13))
 (segment (start 51.53 -29.43) (end 50.04 -27.94) (width 0.25) (layer F.Cu) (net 13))
 (segment (start 47.54 -27.94) (end 47.31 -27.94) (width 0.25) (layer F.Cu) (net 13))
 (segment (start 51.53 -30.48) (end 51.53 -29.43) (width 0.25) (layer F.Cu) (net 13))
 (segment (start 47.31 -27.74) (end 46.24 -26.67) (width 0.25) (layer F.Cu) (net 13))
 (segment (start 47.31 -27.94) (end 47.31 -27.74) (width 0.25) (layer F.Cu) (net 13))
 (segment (start 31.605001 -34.434999) (end 31.279999 -34.760001) (width 0.25) (layer F.Cu) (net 13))
 (segment (start 31.605001 -32.249997) (end 31.605001 -34.434999) (width 0.25) (layer F.Cu) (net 13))
 (segment (start 31.279999 -34.760001) (end 30.48 -35.56) (width 0.25) (layer F.Cu) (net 13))
 (segment (start 37.184998 -26.67) (end 31.605001 -32.249997) (width 0.25) (layer F.Cu) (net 13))
 (segment (start 46.24 -26.67) (end 37.184998 -26.67) (width 0.25) (layer F.Cu) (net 13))
 (segment (start 49.53 -52.39) (end 49.53 -58.42) (width 0.25) (layer F.Cu) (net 24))
 (segment (start 49.53 -38.42) (end 49.53 -45.72) (width 0.25) (layer F.Cu) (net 23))
 (segment (start 49.53 -45.72) (end 49.53 -51.75) (width 0.25) (layer F.Cu) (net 23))
 (segment (start 36.4975 -40.64) (end 38.1 -40.64) (width 0.25) (layer B.Cu) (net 9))
 (segment (start 36.4975 -38.1) (end 38.1 -38.1) (width 0.25) (layer B.Cu) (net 7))
 (segment (start 36.4975 -35.56) (end 38.1 -35.56) (width 0.25) (layer B.Cu) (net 5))
 (segment (start 36.4975 -50.8) (end 38.1 -50.8) (width 0.25) (layer B.Cu) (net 3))
 (segment (start 40 -50.8) (end 40.64 -50.16) (width 0.25) (layer B.Cu) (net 3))
 (segment (start 38.1 -50.8) (end 40 -50.8) (width 0.25) (layer B.Cu) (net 3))
 (segment (start 40.64 -48.26) (end 38.1 -48.26) (width 0.25) (layer B.Cu) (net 4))
 (segment (start 36.4975 -48.26) (end 38.1 -48.26) (width 0.25) (layer B.Cu) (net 4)))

